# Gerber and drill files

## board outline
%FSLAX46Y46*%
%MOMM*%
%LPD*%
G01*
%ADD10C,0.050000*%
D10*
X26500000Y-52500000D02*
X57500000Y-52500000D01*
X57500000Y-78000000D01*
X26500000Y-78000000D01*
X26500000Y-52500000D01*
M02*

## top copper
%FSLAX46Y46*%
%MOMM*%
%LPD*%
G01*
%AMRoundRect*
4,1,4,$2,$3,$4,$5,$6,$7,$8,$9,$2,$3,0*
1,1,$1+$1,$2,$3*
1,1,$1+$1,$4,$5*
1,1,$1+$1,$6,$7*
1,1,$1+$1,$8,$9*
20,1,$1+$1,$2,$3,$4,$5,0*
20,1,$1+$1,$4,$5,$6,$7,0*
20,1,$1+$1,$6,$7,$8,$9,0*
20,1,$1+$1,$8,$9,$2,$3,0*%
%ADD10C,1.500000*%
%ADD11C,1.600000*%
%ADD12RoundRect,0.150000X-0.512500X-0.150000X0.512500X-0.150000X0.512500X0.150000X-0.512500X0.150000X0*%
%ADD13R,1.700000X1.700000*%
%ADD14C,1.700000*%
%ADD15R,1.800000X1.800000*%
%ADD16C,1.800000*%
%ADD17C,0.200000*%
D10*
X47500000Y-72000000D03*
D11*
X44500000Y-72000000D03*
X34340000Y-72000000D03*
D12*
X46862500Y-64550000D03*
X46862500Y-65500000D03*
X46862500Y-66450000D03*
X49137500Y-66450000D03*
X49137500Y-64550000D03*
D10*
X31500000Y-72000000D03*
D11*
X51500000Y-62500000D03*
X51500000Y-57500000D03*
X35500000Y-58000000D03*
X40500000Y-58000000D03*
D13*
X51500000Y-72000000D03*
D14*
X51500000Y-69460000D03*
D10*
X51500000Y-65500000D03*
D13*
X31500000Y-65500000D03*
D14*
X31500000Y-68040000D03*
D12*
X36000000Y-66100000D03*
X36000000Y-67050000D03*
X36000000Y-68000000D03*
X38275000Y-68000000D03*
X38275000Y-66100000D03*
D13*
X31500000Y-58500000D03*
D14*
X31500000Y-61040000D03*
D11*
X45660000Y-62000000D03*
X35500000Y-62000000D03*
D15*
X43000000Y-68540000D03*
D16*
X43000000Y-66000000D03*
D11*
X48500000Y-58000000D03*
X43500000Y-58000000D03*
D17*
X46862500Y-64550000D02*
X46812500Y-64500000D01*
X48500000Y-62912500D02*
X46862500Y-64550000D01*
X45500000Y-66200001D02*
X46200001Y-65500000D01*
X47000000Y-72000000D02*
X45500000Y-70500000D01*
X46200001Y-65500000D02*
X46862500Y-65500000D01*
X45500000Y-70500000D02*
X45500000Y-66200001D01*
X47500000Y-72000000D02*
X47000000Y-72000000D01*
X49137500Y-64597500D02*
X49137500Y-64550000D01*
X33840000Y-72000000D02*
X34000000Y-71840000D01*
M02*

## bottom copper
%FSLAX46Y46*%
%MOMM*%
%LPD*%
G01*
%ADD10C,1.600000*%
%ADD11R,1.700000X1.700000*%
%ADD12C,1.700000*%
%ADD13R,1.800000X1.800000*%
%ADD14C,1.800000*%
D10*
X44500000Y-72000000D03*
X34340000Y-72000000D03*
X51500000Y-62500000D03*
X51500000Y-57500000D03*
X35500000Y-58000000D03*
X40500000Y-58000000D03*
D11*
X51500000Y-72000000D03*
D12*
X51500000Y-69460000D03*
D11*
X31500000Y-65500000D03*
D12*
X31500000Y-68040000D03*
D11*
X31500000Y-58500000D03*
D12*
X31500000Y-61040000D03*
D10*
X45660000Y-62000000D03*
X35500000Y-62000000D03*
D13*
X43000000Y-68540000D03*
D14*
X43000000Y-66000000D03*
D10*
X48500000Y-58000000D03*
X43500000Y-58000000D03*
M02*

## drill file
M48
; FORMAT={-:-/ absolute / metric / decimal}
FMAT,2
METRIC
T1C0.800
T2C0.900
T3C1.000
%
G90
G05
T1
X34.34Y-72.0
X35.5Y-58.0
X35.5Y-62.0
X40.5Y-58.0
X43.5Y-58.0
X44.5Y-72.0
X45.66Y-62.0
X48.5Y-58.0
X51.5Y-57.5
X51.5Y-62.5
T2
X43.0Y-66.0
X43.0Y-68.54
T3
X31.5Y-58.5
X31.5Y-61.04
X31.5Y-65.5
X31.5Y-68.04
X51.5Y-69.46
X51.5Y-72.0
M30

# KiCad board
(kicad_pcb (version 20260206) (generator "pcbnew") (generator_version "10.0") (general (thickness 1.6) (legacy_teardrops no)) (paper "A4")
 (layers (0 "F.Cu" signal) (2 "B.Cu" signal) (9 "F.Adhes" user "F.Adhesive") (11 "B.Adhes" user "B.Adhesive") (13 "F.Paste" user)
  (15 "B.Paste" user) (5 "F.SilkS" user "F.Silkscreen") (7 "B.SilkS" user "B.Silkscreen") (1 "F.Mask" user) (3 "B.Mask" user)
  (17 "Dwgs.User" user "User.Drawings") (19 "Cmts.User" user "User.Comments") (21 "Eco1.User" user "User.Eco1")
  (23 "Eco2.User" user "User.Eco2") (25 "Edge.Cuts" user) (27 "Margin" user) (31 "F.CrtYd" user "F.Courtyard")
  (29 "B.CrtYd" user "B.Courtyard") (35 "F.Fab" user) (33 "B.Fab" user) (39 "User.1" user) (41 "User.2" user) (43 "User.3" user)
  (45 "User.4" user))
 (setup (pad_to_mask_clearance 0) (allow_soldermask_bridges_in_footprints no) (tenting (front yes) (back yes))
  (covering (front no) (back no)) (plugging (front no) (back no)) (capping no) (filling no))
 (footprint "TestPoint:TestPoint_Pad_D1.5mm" (layer "F.Cu") (at 47.5 72)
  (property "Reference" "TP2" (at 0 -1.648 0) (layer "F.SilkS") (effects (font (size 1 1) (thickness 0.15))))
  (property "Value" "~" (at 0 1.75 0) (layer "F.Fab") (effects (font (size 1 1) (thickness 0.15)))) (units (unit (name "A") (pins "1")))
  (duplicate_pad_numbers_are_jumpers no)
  (pad "1" smd circle (at 0 0) (size 1.5 1.5) (layers "F.Cu" "F.Mask") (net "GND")))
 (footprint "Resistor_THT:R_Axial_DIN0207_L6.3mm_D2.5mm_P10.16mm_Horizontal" (layer "F.Cu") (at 44.5 72 180)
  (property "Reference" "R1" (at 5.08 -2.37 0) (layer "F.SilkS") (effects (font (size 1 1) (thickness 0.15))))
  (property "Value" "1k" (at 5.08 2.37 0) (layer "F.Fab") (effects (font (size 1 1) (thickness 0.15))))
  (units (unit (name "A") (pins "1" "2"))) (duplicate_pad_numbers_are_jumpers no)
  (pad "1" thru_hole circle (at 0 0 180) (size 1.6 1.6) (drill 0.8) (layers "*.Cu" "*.Mask") (remove_unused_layers no) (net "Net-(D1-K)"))
  (pad "2" thru_hole circle (at 10.16 0 180) (size 1.6 1.6) (drill 0.8) (layers "*.Cu" "*.Mask") (remove_unused_layers no)
   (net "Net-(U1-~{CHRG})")))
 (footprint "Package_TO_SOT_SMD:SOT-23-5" (layer "F.Cu") (at 48 65.5)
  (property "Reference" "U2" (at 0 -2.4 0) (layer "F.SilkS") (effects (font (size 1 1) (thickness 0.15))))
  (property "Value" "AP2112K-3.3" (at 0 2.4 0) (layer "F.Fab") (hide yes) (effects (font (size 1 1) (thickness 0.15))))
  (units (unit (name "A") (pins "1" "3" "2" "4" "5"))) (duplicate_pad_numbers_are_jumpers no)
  (pad "1" smd roundrect (at -1.1375 -0.95) (size 1.325 0.6) (layers "F.Cu" "F.Mask" "F.Paste") (roundrect_rratio 0.25)
   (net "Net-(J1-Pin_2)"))
  (pad "2" smd roundrect (at -1.1375 0) (size 1.325 0.6) (layers "F.Cu" "F.Mask" "F.Paste") (roundrect_rratio 0.25) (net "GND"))
  (pad "3" smd roundrect (at -1.1375 0.95) (size 1.325 0.6) (layers "F.Cu" "F.Mask" "F.Paste") (roundrect_rratio 0.25)
   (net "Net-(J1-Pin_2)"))
  (pad "4" smd roundrect (at 1.1375 0.95) (size 1.325 0.6) (layers "F.Cu" "F.Mask" "F.Paste") (roundrect_rratio 0.25)
   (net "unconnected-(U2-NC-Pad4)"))
  (pad "5" smd roundrect (at 1.1375 -0.95) (size 1.325 0.6) (layers "F.Cu" "F.Mask" "F.Paste") (roundrect_rratio 0.25)
   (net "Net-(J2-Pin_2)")))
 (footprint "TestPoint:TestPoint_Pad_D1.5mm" (layer "F.Cu") (at 31.5 72)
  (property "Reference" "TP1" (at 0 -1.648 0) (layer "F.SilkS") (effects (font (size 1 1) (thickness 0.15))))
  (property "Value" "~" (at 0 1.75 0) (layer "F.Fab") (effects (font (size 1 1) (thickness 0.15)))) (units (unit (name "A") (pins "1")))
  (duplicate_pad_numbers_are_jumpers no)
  (pad "1" smd circle (at 0 0) (size 1.5 1.5) (layers "F.Cu" "F.Mask") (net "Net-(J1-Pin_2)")))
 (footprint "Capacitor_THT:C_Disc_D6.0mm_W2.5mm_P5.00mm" (layer "F.Cu") (at 51.5 62.5 90)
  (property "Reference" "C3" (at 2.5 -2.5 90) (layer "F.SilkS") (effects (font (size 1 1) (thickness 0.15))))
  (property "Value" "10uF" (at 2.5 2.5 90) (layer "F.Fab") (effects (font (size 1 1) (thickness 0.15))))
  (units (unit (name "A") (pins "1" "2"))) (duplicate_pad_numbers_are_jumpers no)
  (pad "1" thru_hole circle (at 0 0 90) (size 1.6 1.6) (drill 0.8) (layers "*.Cu" "*.Mask") (remove_unused_layers no) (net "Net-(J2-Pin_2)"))
  (pad "2" thru_hole circle (at 5 0 90) (size 1.6 1.6) (drill 0.8) (layers "*.Cu" "*.Mask") (remove_unused_layers no) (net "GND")))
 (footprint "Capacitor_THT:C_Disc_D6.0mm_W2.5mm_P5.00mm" (layer "F.Cu") (at 35.5 58)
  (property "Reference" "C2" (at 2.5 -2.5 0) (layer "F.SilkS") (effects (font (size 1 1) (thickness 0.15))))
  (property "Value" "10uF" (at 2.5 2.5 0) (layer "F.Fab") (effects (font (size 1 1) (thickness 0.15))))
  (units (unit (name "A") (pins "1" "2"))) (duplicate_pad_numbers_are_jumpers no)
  (pad "1" thru_hole circle (at 0 0) (size 1.6 1.6) (drill 0.8) (layers "*.Cu" "*.Mask") (remove_unused_layers no) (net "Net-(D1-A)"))
  (pad "2" thru_hole circle (at 5 0) (size 1.6 1.6) (drill 0.8) (layers "*.Cu" "*.Mask") (remove_unused_layers no) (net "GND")))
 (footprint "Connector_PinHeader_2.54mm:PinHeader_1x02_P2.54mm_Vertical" (layer "F.Cu") (at 51.5 72 180)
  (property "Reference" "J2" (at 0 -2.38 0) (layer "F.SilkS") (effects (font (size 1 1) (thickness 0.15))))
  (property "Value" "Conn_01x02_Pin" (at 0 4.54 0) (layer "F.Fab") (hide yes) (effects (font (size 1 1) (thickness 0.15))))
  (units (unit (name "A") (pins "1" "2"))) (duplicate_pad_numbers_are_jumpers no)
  (pad "1" thru_hole rect (at 0 0 180) (size 1.7 1.7) (drill 1) (layers "*.Cu" "*.Mask") (remove_unused_layers no) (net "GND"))
  (pad "2" thru_hole circle (at 0 2.54 180) (size 1.7 1.7) (drill 1) (layers "*.Cu" "*.Mask") (remove_unused_layers no)
   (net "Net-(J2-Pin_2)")))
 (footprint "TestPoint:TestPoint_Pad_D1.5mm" (layer "F.Cu") (at 51.5 65.5)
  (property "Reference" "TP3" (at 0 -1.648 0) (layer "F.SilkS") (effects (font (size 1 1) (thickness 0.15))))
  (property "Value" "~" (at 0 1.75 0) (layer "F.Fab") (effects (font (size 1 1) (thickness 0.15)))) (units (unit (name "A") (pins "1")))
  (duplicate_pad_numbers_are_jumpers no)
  (pad "1" smd circle (at 0 0) (size 1.5 1.5) (layers "F.Cu" "F.Mask") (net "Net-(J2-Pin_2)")))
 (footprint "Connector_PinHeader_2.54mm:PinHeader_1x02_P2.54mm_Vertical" (layer "F.Cu") (at 31.5 65.5)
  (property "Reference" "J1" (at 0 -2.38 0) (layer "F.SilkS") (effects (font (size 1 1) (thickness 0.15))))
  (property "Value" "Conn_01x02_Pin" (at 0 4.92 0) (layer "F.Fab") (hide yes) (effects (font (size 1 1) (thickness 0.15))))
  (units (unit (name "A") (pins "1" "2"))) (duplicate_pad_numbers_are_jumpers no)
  (pad "1" thru_hole rect (at 0 0) (size 1.7 1.7) (drill 1) (layers "*.Cu" "*.Mask") (remove_unused_layers no) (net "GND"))
  (pad "2" thru_hole circle (at 0 2.54) (size 1.7 1.7) (drill 1) (layers "*.Cu" "*.Mask") (remove_unused_layers no) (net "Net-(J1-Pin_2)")))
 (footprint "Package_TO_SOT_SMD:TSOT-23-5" (layer "F.Cu") (at 37.1375 67.05)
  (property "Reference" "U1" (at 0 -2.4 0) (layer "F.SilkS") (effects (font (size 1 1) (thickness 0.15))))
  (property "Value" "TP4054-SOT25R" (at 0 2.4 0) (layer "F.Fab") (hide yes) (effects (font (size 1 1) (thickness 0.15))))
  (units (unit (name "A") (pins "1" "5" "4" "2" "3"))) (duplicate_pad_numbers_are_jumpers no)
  (pad "1" smd roundrect (at -1.1375 -0.95) (size 1.325 0.6) (layers "F.Cu" "F.Mask" "F.Paste") (roundrect_rratio 0.25)
   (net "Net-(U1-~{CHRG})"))
  (pad "2" smd roundrect (at -1.1375 0) (size 1.325 0.6) (layers "F.Cu" "F.Mask" "F.Paste") (roundrect_rratio 0.25) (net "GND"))
  (pad "3" smd roundrect (at -1.1375 0.95) (size 1.325 0.6) (layers "F.Cu" "F.Mask" "F.Paste") (roundrect_rratio 0.25)
   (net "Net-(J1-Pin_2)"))
  (pad "4" smd roundrect (at 1.1375 0.95) (size 1.325 0.6) (layers "F.Cu" "F.Mask" "F.Paste") (roundrect_rratio 0.25) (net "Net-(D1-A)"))
  (pad "5" smd roundrect (at 1.1375 -0.95) (size 1.325 0.6) (layers "F.Cu" "F.Mask" "F.Paste") (roundrect_rratio 0.25) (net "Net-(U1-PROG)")))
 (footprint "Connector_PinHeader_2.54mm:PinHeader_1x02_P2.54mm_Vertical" (layer "F.Cu") (at 31.5 58.5)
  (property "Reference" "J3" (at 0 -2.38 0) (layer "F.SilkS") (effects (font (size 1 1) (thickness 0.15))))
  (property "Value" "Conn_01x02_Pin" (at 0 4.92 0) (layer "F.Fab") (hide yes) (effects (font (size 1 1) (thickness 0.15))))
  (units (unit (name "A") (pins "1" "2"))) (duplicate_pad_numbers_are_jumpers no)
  (pad "1" thru_hole rect (at 0 0) (size 1.7 1.7) (drill 1) (layers "*.Cu" "*.Mask") (remove_unused_layers no) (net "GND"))
  (pad "2" thru_hole circle (at 0 2.54) (size 1.7 1.7) (drill 1) (layers "*.Cu" "*.Mask") (remove_unused_layers no) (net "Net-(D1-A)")))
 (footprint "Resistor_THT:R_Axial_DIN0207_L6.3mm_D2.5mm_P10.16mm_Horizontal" (layer "F.Cu") (at 45.66 62 180)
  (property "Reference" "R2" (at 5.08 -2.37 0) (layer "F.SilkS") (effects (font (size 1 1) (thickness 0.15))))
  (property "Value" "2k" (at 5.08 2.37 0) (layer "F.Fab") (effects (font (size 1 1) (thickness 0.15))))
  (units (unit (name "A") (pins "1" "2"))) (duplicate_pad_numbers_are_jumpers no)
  (pad "1" thru_hole circle (at 0 0 180) (size 1.6 1.6) (drill 0.8) (layers "*.Cu" "*.Mask") (remove_unused_layers no) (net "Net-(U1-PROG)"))
  (pad "2" thru_hole circle (at 10.16 0 180) (size 1.6 1.6) (drill 0.8) (layers "*.Cu" "*.Mask") (remove_unused_layers no) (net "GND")))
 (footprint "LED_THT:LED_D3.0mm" (layer "F.Cu") (at 43 68.54 90)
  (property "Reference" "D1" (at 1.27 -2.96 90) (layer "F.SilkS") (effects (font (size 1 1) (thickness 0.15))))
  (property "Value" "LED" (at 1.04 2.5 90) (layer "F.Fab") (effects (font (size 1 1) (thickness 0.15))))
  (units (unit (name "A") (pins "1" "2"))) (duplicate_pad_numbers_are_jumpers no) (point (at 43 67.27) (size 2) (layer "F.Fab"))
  (pad "1" thru_hole rect (at 0 0 90) (size 1.8 1.8) (drill 0.9) (layers "*.Cu" "*.Mask") (remove_unused_layers no) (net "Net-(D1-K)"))
  (pad "2" thru_hole circle (at 2.54 0 90) (size 1.8 1.8) (drill 0.9) (layers "*.Cu" "*.Mask") (remove_unused_layers no) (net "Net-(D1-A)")))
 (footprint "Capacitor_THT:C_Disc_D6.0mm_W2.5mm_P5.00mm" (layer "F.Cu") (at 48.5 58 180)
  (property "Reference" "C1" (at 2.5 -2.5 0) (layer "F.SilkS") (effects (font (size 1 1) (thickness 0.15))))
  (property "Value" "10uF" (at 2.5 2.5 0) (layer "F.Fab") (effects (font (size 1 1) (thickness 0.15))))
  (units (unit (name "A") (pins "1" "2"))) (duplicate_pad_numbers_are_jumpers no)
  (pad "1" thru_hole circle (at 0 0 180) (size 1.6 1.6) (drill 0.8) (layers "*.Cu" "*.Mask") (remove_unused_layers no)
   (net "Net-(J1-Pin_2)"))
  (pad "2" thru_hole circle (at 5 0 180) (size 1.6 1.6) (drill 0.8) (layers "*.Cu" "*.Mask") (remove_unused_layers no) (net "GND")))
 (gr_rect (start 26.5 52.5) (end 57.5 78) (stroke (width 0.05) (type default)) (fill no) (layer "Edge.Cuts"))
 (segment (start 46.8625 64.55) (end 46.8125 64.5) (width 0.2) (layer "F.Cu") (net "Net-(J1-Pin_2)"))
 (segment (start 48.5 62.9125) (end 46.8625 64.55) (width 0.2) (layer "F.Cu") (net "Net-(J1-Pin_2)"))
 (segment (start 45.5 66.200001) (end 46.200001 65.5) (width 0.2) (layer "F.Cu") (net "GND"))
 (segment (start 47 72) (end 45.5 70.5) (width 0.2) (layer "F.Cu") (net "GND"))
 (segment (start 46.200001 65.5) (end 46.8625 65.5) (width 0.2) (layer "F.Cu") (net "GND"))
 (segment (start 45.5 70.5) (end 45.5 66.200001) (width 0.2) (layer "F.Cu") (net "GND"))
 (segment (start 47.5 72) (end 47 72) (width 0.2) (layer "F.Cu") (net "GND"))
 (segment (start 49.1375 64.5975) (end 49.1375 64.55) (width 0.2) (layer "F.Cu") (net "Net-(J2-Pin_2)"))
 (segment (start 33.84 72) (end 34 71.84) (width 0.2) (layer "F.Cu") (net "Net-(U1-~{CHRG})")))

